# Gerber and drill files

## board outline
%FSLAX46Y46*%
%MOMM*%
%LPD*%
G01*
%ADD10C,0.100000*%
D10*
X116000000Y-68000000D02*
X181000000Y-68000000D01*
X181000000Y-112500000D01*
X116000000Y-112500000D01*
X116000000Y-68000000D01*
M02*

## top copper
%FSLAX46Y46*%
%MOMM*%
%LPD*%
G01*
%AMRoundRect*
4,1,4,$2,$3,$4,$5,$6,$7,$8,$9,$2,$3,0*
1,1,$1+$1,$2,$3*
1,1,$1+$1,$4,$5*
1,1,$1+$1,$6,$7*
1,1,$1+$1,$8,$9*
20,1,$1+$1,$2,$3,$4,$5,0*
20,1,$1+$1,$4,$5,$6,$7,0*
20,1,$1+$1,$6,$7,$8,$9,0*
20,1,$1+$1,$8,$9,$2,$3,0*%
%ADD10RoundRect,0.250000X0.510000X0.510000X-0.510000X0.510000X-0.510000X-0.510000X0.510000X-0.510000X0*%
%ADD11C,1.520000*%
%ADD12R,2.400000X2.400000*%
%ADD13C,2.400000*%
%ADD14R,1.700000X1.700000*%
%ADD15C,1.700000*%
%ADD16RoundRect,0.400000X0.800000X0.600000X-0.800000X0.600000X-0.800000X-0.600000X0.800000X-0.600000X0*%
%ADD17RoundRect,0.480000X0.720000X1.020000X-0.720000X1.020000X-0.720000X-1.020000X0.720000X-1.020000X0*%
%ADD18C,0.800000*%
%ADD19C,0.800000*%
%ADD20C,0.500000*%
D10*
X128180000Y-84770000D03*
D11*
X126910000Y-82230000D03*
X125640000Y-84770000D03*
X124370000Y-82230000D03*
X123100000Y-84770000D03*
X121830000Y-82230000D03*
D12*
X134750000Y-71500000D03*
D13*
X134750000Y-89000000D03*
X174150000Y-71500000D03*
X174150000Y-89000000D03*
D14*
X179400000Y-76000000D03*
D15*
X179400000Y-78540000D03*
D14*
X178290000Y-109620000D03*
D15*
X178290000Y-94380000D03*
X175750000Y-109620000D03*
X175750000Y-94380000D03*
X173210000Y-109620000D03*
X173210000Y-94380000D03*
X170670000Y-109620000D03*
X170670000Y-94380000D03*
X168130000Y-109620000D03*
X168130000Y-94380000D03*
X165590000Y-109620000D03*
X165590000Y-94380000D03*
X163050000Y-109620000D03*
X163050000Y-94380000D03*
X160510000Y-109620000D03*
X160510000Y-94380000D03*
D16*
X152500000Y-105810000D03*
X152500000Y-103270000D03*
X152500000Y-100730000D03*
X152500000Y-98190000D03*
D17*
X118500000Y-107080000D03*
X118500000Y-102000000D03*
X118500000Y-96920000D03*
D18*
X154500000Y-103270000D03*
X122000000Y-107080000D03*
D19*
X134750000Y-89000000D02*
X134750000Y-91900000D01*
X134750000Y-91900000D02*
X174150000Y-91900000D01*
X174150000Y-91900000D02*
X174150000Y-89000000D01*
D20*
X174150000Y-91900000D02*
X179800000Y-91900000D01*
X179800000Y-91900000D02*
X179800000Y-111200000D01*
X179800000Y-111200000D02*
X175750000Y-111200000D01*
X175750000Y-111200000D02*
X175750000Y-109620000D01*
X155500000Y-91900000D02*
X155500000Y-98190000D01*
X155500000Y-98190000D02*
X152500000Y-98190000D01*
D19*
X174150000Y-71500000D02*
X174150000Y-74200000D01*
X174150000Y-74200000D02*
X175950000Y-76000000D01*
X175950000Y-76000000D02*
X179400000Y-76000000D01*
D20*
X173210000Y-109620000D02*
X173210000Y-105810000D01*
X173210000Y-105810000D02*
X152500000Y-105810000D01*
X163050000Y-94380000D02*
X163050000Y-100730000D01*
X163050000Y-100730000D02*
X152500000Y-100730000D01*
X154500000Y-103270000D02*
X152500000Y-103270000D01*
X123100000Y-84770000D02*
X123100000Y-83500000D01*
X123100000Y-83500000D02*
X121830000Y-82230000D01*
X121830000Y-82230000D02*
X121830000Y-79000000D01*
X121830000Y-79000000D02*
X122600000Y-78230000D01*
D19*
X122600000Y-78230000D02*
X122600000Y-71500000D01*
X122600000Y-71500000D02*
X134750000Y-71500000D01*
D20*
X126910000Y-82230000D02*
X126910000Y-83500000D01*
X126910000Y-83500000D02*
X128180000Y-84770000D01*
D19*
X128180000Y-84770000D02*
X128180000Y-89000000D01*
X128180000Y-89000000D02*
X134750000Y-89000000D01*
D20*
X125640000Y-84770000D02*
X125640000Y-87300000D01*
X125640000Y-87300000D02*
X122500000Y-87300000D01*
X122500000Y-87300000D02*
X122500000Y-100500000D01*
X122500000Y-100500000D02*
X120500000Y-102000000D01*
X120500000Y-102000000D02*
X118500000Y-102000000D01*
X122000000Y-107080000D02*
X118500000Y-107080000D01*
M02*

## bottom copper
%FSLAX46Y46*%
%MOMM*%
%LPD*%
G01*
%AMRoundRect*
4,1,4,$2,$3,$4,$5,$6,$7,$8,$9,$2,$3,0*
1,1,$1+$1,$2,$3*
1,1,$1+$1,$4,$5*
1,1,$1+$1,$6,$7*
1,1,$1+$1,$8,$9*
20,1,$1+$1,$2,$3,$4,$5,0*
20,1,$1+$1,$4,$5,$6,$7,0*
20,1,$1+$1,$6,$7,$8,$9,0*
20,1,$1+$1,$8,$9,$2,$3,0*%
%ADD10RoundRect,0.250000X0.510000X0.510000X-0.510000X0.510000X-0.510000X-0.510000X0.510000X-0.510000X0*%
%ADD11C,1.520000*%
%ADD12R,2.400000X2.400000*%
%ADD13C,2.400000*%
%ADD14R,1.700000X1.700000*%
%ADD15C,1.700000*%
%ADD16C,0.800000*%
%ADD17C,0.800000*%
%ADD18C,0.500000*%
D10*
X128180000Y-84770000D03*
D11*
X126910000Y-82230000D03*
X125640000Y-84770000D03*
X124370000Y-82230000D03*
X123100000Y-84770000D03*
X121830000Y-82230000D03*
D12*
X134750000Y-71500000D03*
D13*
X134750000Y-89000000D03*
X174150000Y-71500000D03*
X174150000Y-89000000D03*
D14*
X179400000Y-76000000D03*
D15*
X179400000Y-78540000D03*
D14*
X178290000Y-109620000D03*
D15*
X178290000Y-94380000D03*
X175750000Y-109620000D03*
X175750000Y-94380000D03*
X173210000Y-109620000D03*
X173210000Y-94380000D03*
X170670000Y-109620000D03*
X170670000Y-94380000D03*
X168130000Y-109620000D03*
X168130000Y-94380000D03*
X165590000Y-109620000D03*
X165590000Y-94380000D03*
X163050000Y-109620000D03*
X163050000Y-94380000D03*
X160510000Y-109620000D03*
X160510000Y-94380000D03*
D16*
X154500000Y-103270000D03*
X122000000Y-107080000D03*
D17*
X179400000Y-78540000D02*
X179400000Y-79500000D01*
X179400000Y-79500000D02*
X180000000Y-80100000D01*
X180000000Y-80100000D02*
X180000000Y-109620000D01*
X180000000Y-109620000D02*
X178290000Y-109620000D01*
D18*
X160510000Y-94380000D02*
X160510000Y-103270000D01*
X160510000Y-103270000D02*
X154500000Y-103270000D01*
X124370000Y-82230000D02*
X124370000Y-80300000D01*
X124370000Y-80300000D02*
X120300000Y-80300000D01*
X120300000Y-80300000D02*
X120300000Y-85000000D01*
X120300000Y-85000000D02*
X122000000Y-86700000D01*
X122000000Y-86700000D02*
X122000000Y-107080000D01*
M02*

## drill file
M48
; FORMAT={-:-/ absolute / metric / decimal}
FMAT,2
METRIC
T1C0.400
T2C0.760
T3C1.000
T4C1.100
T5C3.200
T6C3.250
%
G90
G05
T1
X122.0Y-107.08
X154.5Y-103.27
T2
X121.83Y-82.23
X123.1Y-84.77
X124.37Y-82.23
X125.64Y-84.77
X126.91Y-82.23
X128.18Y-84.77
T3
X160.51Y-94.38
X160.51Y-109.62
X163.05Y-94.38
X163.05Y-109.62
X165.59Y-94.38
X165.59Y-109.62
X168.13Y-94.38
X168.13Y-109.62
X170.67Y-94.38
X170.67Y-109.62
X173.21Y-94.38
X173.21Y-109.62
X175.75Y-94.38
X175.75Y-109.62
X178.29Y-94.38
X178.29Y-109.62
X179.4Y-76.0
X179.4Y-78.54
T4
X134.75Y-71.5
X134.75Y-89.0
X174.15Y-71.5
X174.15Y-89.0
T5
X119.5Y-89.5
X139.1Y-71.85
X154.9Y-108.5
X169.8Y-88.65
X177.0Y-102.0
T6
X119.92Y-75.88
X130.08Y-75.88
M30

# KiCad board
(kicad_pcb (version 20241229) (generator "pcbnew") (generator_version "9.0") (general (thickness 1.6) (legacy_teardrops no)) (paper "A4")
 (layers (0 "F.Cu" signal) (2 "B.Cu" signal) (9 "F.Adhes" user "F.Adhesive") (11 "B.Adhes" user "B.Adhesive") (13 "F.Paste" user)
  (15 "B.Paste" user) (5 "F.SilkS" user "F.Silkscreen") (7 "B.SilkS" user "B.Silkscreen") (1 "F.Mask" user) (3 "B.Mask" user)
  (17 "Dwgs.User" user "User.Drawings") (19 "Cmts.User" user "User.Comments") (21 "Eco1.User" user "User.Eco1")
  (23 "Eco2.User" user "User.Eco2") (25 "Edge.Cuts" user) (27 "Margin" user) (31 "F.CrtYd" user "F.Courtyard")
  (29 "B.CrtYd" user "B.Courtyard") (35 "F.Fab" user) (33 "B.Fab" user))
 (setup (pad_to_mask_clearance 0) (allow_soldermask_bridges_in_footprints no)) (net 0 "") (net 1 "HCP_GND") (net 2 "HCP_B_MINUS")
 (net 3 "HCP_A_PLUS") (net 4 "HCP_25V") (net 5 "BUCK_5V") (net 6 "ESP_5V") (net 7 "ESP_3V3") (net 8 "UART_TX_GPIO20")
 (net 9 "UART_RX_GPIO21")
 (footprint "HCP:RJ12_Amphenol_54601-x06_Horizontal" (layer "F.Cu") (at 128.18 84.77 180)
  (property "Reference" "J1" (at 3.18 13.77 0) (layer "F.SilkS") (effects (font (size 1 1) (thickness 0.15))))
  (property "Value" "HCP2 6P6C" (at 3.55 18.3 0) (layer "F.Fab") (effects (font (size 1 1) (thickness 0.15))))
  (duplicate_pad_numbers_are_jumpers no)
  (pad "" np_thru_hole circle (at -1.9 8.89 180) (size 3.25 3.25) (drill 3.25) (layers "*.Cu" "*.Mask"))
  (pad "" np_thru_hole circle (at 8.26 8.89 180) (size 3.25 3.25) (drill 3.25) (layers "*.Cu" "*.Mask"))
  (pad "1" thru_hole roundrect (at 0 0 180) (size 1.52 1.52) (drill 0.76) (layers "*.Cu" "*.Mask") (remove_unused_layers no)
   (roundrect_rratio 0.1644736842) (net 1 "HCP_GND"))
  (pad "2" thru_hole circle (at 1.27 2.54 180) (size 1.52 1.52) (drill 0.76) (layers "*.Cu" "*.Mask") (remove_unused_layers no)
   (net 1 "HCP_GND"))
  (pad "3" thru_hole circle (at 2.54 0 180) (size 1.52 1.52) (drill 0.76) (layers "*.Cu" "*.Mask") (remove_unused_layers no)
   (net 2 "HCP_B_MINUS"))
  (pad "4" thru_hole circle (at 3.81 2.54 180) (size 1.52 1.52) (drill 0.76) (layers "*.Cu" "*.Mask") (remove_unused_layers no)
   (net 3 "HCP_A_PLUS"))
  (pad "5" thru_hole circle (at 5.08 0 180) (size 1.52 1.52) (drill 0.76) (layers "*.Cu" "*.Mask") (remove_unused_layers no)
   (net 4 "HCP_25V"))
  (pad "6" thru_hole circle (at 6.35 2.54 180) (size 1.52 1.52) (drill 0.76) (layers "*.Cu" "*.Mask") (remove_unused_layers no)
   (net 4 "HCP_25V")))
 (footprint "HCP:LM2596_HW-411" (layer "F.Cu") (at 154.45 80.25 0)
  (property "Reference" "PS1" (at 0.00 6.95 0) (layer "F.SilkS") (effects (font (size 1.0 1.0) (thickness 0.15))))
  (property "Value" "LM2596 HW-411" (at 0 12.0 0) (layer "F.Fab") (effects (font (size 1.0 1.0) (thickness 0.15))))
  (pad "1" thru_hole rect (at -19.7 -8.75) (size 2.4 2.4) (drill 1.1) (layers "*.Cu" "*.Mask") (remove_unused_layers no) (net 4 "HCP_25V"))
  (pad "2" thru_hole circle (at -19.7 8.75) (size 2.4 2.4) (drill 1.1) (layers "*.Cu" "*.Mask") (remove_unused_layers no) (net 1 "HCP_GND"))
  (pad "3" thru_hole circle (at 19.7 -8.75) (size 2.4 2.4) (drill 1.1) (layers "*.Cu" "*.Mask") (remove_unused_layers no) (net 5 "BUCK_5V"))
  (pad "4" thru_hole circle (at 19.7 8.75) (size 2.4 2.4) (drill 1.1) (layers "*.Cu" "*.Mask") (remove_unused_layers no) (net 1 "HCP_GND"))
  (pad "" np_thru_hole circle (at -15.35 -8.4) (size 3.2 3.2) (drill 3.2) (layers "*.Cu" "*.Mask"))
  (pad "" np_thru_hole circle (at 15.35 8.4) (size 3.2 3.2) (drill 3.2) (layers "*.Cu" "*.Mask")))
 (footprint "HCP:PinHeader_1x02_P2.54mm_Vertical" (layer "F.Cu") (at 179.4 76.0 0)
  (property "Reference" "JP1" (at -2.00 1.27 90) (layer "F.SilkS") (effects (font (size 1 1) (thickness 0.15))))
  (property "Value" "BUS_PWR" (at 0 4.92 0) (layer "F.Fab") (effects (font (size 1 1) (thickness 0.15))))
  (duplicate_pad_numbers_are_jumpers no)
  (pad "1" thru_hole rect (at 0 0) (size 1.7 1.7) (drill 1) (layers "*.Cu" "*.Mask") (remove_unused_layers no) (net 5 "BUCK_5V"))
  (pad "2" thru_hole circle (at 0 2.54) (size 1.7 1.7) (drill 1) (layers "*.Cu" "*.Mask") (remove_unused_layers no) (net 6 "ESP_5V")))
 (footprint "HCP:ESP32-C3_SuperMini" (layer "F.Cu") (at 169.4 102.0 270)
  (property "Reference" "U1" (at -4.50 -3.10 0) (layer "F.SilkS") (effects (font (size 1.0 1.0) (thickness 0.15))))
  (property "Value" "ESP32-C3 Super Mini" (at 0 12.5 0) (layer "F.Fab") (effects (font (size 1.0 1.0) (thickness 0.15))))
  (pad "1" thru_hole rect (at 7.62 -8.89 270) (size 1.7 1.7) (drill 1.0) (layers "*.Cu" "*.Mask") (remove_unused_layers no) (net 6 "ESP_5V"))
  (pad "2" thru_hole circle (at -7.62 -8.89 270) (size 1.7 1.7) (drill 1.0) (layers "*.Cu" "*.Mask") (remove_unused_layers no))
  (pad "3" thru_hole circle (at 7.62 -6.35 270) (size 1.7 1.7) (drill 1.0) (layers "*.Cu" "*.Mask") (remove_unused_layers no)
   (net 1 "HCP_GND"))
  (pad "4" thru_hole circle (at -7.62 -6.35 270) (size 1.7 1.7) (drill 1.0) (layers "*.Cu" "*.Mask") (remove_unused_layers no))
  (pad "5" thru_hole circle (at 7.62 -3.81 270) (size 1.7 1.7) (drill 1.0) (layers "*.Cu" "*.Mask") (remove_unused_layers no)
   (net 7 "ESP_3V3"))
  (pad "6" thru_hole circle (at -7.62 -3.81 270) (size 1.7 1.7) (drill 1.0) (layers "*.Cu" "*.Mask") (remove_unused_layers no))
  (pad "7" thru_hole circle (at 7.62 -1.27 270) (size 1.7 1.7) (drill 1.0) (layers "*.Cu" "*.Mask") (remove_unused_layers no))
  (pad "8" thru_hole circle (at -7.62 -1.27 270) (size 1.7 1.7) (drill 1.0) (layers "*.Cu" "*.Mask") (remove_unused_layers no))
  (pad "9" thru_hole circle (at 7.62 1.27 270) (size 1.7 1.7) (drill 1.0) (layers "*.Cu" "*.Mask") (remove_unused_layers no))
  (pad "10" thru_hole circle (at -7.62 1.27 270) (size 1.7 1.7) (drill 1.0) (layers "*.Cu" "*.Mask") (remove_unused_layers no))
  (pad "11" thru_hole circle (at 7.62 3.81 270) (size 1.7 1.7) (drill 1.0) (layers "*.Cu" "*.Mask") (remove_unused_layers no))
  (pad "12" thru_hole circle (at -7.62 3.81 270) (size 1.7 1.7) (drill 1.0) (layers "*.Cu" "*.Mask") (remove_unused_layers no))
  (pad "13" thru_hole circle (at 7.62 6.35 270) (size 1.7 1.7) (drill 1.0) (layers "*.Cu" "*.Mask") (remove_unused_layers no))
  (pad "14" thru_hole circle (at -7.62 6.35 270) (size 1.7 1.7) (drill 1.0) (layers "*.Cu" "*.Mask") (remove_unused_layers no)
   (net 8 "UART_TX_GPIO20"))
  (pad "15" thru_hole circle (at 7.62 8.89 270) (size 1.7 1.7) (drill 1.0) (layers "*.Cu" "*.Mask") (remove_unused_layers no))
  (pad "16" thru_hole circle (at -7.62 8.89 270) (size 1.7 1.7) (drill 1.0) (layers "*.Cu" "*.Mask") (remove_unused_layers no)
   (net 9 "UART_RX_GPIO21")))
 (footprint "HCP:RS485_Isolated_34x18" (layer "F.Cu") (at 135.5 102.0 180)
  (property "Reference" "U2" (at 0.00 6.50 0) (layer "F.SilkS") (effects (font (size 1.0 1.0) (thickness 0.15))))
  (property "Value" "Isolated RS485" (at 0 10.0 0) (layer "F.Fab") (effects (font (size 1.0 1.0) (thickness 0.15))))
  (pad "1" smd roundrect (at -17 -3.81 180) (size 2.4 2.0) (layers "F.Cu" "F.Paste" "F.Mask") (roundrect_rratio 0.2) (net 7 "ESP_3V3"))
  (pad "2" smd roundrect (at -17 -1.27 180) (size 2.4 2.0) (layers "F.Cu" "F.Paste" "F.Mask") (roundrect_rratio 0.2)
   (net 9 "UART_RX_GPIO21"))
  (pad "3" smd roundrect (at -17 1.27 180) (size 2.4 2.0) (layers "F.Cu" "F.Paste" "F.Mask") (roundrect_rratio 0.2) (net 8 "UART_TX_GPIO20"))
  (pad "4" smd roundrect (at -17 3.81 180) (size 2.4 2.0) (layers "F.Cu" "F.Paste" "F.Mask") (roundrect_rratio 0.2) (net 1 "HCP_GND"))
  (pad "5" smd roundrect (at 17 -5.08 180) (size 2.4 3.0) (layers "F.Cu" "F.Paste" "F.Mask") (roundrect_rratio 0.2) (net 3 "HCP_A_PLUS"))
  (pad "6" smd roundrect (at 17 0 180) (size 2.4 3.0) (layers "F.Cu" "F.Paste" "F.Mask") (roundrect_rratio 0.2) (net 2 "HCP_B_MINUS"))
  (pad "7" smd roundrect (at 17 5.08 180) (size 2.4 3.0) (layers "F.Cu" "F.Paste" "F.Mask") (roundrect_rratio 0.2)))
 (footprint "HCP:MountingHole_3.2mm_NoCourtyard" (layer "F.Cu") (at 119.5 89.5 0)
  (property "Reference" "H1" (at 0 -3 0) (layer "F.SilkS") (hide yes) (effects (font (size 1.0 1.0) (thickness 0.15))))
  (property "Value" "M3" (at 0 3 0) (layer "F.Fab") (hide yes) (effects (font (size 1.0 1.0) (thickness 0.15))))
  (pad "" np_thru_hole circle (at 0 0) (size 3.2 3.2) (drill 3.2) (layers "*.Cu" "*.Mask")))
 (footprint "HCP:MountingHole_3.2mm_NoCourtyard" (layer "F.Cu") (at 154.9 108.5 0)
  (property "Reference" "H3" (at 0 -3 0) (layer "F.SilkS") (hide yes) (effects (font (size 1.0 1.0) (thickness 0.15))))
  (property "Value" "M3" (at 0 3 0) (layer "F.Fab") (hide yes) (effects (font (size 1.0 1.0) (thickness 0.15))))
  (pad "" np_thru_hole circle (at 0 0) (size 3.2 3.2) (drill 3.2) (layers "*.Cu" "*.Mask")))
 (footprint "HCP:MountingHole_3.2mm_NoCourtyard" (layer "F.Cu") (at 177.0 102.0 0)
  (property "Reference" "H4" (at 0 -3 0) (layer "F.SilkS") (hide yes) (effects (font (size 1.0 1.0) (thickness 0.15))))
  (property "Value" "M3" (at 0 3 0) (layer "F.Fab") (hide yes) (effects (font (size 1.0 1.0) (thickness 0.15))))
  (pad "" np_thru_hole circle (at 0 0) (size 3.2 3.2) (drill 3.2) (layers "*.Cu" "*.Mask")))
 (segment (start 134.75 89.0) (end 134.75 91.9) (width 0.8) (layer "F.Cu") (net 1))
 (segment (start 134.75 91.9) (end 174.15 91.9) (width 0.8) (layer "F.Cu") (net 1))
 (segment (start 174.15 91.9) (end 174.15 89.0) (width 0.8) (layer "F.Cu") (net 1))
 (segment (start 174.15 91.9) (end 179.8 91.9) (width 0.5) (layer "F.Cu") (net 1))
 (segment (start 179.8 91.9) (end 179.8 111.2) (width 0.5) (layer "F.Cu") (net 1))
 (segment (start 179.8 111.2) (end 175.75 111.2) (width 0.5) (layer "F.Cu") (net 1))
 (segment (start 175.75 111.2) (end 175.75 109.62) (width 0.5) (layer "F.Cu") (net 1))
 (segment (start 155.5 91.9) (end 155.5 98.19) (width 0.5) (layer "F.Cu") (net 1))
 (segment (start 155.5 98.19) (end 152.5 98.19) (width 0.5) (layer "F.Cu") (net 1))
 (segment (start 174.15 71.5) (end 174.15 74.2) (width 0.8) (layer "F.Cu") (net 5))
 (segment (start 174.15 74.2) (end 175.95 76.0) (width 0.8) (layer "F.Cu") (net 5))
 (segment (start 175.95 76.0) (end 179.4 76.0) (width 0.8) (layer "F.Cu") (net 5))
 (segment (start 179.4 78.54) (end 179.4 79.5) (width 0.8) (layer "B.Cu") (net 6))
 (segment (start 179.4 79.5) (end 180.0 80.1) (width 0.8) (layer "B.Cu") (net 6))
 (segment (start 180.0 80.1) (end 180.0 109.62) (width 0.8) (layer "B.Cu") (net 6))
 (segment (start 180.0 109.62) (end 178.29 109.62) (width 0.8) (layer "B.Cu") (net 6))
 (segment (start 173.21 109.62) (end 173.21 105.81) (width 0.5) (layer "F.Cu") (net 7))
 (segment (start 173.21 105.81) (end 152.5 105.81) (width 0.5) (layer "F.Cu") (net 7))
 (segment (start 163.05 94.38) (end 163.05 100.73) (width 0.5) (layer "F.Cu") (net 8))
 (segment (start 163.05 100.73) (end 152.5 100.73) (width 0.5) (layer "F.Cu") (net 8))
 (segment (start 160.51 94.38) (end 160.51 103.27) (width 0.5) (layer "B.Cu") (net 9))
 (segment (start 160.51 103.27) (end 154.5 103.27) (width 0.5) (layer "B.Cu") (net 9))
 (segment (start 154.5 103.27) (end 152.5 103.27) (width 0.5) (layer "F.Cu") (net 9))
 (segment (start 123.1 84.77) (end 123.1 83.5) (width 0.5) (layer "F.Cu") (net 4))
 (segment (start 123.1 83.5) (end 121.83 82.23) (width 0.5) (layer "F.Cu") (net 4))
 (segment (start 121.83 82.23) (end 121.83 79.0) (width 0.5) (layer "F.Cu") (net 4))
 (segment (start 121.83 79.0) (end 122.6 78.23) (width 0.5) (layer "F.Cu") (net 4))
 (segment (start 122.6 78.23) (end 122.6 71.5) (width 0.8) (layer "F.Cu") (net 4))
 (segment (start 122.6 71.5) (end 134.75 71.5) (width 0.8) (layer "F.Cu") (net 4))
 (segment (start 126.91 82.23) (end 126.91 83.5) (width 0.5) (layer "F.Cu") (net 1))
 (segment (start 126.91 83.5) (end 128.18 84.77) (width 0.5) (layer "F.Cu") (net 1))
 (segment (start 128.18 84.77) (end 128.18 89.0) (width 0.8) (layer "F.Cu") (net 1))
 (segment (start 128.18 89.0) (end 134.75 89.0) (width 0.8) (layer "F.Cu") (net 1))
 (segment (start 125.64 84.77) (end 125.64 87.3) (width 0.5) (layer "F.Cu") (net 2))
 (segment (start 125.64 87.3) (end 122.5 87.3) (width 0.5) (layer "F.Cu") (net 2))
 (segment (start 122.5 87.3) (end 122.5 100.5) (width 0.5) (layer "F.Cu") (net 2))
 (segment (start 122.5 100.5) (end 120.5 102.0) (width 0.5) (layer "F.Cu") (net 2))
 (segment (start 120.5 102.0) (end 118.5 102.0) (width 0.5) (layer "F.Cu") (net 2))
 (segment (start 124.37 82.23) (end 124.37 80.3) (width 0.5) (layer "B.Cu") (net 3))
 (segment (start 124.37 80.3) (end 120.3 80.3) (width 0.5) (layer "B.Cu") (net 3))
 (segment (start 120.3 80.3) (end 120.3 85.0) (width 0.5) (layer "B.Cu") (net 3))
 (segment (start 120.3 85.0) (end 122.0 86.7) (width 0.5) (layer "B.Cu") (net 3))
 (segment (start 122.0 86.7) (end 122.0 107.08) (width 0.5) (layer "B.Cu") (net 3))
 (segment (start 122.0 107.08) (end 118.5 107.08) (width 0.5) (layer "F.Cu") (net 3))
 (via (at 154.5 103.27) (size 0.8) (drill 0.4) (layers "F.Cu" "B.Cu") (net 9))
 (via (at 122.0 107.08) (size 0.8) (drill 0.4) (layers "F.Cu" "B.Cu") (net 3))
 (gr_rect (start 116.0 68.0) (end 181.0 112.5) (stroke (width 0.1) (type default)) (fill none) (layer "Edge.Cuts")))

